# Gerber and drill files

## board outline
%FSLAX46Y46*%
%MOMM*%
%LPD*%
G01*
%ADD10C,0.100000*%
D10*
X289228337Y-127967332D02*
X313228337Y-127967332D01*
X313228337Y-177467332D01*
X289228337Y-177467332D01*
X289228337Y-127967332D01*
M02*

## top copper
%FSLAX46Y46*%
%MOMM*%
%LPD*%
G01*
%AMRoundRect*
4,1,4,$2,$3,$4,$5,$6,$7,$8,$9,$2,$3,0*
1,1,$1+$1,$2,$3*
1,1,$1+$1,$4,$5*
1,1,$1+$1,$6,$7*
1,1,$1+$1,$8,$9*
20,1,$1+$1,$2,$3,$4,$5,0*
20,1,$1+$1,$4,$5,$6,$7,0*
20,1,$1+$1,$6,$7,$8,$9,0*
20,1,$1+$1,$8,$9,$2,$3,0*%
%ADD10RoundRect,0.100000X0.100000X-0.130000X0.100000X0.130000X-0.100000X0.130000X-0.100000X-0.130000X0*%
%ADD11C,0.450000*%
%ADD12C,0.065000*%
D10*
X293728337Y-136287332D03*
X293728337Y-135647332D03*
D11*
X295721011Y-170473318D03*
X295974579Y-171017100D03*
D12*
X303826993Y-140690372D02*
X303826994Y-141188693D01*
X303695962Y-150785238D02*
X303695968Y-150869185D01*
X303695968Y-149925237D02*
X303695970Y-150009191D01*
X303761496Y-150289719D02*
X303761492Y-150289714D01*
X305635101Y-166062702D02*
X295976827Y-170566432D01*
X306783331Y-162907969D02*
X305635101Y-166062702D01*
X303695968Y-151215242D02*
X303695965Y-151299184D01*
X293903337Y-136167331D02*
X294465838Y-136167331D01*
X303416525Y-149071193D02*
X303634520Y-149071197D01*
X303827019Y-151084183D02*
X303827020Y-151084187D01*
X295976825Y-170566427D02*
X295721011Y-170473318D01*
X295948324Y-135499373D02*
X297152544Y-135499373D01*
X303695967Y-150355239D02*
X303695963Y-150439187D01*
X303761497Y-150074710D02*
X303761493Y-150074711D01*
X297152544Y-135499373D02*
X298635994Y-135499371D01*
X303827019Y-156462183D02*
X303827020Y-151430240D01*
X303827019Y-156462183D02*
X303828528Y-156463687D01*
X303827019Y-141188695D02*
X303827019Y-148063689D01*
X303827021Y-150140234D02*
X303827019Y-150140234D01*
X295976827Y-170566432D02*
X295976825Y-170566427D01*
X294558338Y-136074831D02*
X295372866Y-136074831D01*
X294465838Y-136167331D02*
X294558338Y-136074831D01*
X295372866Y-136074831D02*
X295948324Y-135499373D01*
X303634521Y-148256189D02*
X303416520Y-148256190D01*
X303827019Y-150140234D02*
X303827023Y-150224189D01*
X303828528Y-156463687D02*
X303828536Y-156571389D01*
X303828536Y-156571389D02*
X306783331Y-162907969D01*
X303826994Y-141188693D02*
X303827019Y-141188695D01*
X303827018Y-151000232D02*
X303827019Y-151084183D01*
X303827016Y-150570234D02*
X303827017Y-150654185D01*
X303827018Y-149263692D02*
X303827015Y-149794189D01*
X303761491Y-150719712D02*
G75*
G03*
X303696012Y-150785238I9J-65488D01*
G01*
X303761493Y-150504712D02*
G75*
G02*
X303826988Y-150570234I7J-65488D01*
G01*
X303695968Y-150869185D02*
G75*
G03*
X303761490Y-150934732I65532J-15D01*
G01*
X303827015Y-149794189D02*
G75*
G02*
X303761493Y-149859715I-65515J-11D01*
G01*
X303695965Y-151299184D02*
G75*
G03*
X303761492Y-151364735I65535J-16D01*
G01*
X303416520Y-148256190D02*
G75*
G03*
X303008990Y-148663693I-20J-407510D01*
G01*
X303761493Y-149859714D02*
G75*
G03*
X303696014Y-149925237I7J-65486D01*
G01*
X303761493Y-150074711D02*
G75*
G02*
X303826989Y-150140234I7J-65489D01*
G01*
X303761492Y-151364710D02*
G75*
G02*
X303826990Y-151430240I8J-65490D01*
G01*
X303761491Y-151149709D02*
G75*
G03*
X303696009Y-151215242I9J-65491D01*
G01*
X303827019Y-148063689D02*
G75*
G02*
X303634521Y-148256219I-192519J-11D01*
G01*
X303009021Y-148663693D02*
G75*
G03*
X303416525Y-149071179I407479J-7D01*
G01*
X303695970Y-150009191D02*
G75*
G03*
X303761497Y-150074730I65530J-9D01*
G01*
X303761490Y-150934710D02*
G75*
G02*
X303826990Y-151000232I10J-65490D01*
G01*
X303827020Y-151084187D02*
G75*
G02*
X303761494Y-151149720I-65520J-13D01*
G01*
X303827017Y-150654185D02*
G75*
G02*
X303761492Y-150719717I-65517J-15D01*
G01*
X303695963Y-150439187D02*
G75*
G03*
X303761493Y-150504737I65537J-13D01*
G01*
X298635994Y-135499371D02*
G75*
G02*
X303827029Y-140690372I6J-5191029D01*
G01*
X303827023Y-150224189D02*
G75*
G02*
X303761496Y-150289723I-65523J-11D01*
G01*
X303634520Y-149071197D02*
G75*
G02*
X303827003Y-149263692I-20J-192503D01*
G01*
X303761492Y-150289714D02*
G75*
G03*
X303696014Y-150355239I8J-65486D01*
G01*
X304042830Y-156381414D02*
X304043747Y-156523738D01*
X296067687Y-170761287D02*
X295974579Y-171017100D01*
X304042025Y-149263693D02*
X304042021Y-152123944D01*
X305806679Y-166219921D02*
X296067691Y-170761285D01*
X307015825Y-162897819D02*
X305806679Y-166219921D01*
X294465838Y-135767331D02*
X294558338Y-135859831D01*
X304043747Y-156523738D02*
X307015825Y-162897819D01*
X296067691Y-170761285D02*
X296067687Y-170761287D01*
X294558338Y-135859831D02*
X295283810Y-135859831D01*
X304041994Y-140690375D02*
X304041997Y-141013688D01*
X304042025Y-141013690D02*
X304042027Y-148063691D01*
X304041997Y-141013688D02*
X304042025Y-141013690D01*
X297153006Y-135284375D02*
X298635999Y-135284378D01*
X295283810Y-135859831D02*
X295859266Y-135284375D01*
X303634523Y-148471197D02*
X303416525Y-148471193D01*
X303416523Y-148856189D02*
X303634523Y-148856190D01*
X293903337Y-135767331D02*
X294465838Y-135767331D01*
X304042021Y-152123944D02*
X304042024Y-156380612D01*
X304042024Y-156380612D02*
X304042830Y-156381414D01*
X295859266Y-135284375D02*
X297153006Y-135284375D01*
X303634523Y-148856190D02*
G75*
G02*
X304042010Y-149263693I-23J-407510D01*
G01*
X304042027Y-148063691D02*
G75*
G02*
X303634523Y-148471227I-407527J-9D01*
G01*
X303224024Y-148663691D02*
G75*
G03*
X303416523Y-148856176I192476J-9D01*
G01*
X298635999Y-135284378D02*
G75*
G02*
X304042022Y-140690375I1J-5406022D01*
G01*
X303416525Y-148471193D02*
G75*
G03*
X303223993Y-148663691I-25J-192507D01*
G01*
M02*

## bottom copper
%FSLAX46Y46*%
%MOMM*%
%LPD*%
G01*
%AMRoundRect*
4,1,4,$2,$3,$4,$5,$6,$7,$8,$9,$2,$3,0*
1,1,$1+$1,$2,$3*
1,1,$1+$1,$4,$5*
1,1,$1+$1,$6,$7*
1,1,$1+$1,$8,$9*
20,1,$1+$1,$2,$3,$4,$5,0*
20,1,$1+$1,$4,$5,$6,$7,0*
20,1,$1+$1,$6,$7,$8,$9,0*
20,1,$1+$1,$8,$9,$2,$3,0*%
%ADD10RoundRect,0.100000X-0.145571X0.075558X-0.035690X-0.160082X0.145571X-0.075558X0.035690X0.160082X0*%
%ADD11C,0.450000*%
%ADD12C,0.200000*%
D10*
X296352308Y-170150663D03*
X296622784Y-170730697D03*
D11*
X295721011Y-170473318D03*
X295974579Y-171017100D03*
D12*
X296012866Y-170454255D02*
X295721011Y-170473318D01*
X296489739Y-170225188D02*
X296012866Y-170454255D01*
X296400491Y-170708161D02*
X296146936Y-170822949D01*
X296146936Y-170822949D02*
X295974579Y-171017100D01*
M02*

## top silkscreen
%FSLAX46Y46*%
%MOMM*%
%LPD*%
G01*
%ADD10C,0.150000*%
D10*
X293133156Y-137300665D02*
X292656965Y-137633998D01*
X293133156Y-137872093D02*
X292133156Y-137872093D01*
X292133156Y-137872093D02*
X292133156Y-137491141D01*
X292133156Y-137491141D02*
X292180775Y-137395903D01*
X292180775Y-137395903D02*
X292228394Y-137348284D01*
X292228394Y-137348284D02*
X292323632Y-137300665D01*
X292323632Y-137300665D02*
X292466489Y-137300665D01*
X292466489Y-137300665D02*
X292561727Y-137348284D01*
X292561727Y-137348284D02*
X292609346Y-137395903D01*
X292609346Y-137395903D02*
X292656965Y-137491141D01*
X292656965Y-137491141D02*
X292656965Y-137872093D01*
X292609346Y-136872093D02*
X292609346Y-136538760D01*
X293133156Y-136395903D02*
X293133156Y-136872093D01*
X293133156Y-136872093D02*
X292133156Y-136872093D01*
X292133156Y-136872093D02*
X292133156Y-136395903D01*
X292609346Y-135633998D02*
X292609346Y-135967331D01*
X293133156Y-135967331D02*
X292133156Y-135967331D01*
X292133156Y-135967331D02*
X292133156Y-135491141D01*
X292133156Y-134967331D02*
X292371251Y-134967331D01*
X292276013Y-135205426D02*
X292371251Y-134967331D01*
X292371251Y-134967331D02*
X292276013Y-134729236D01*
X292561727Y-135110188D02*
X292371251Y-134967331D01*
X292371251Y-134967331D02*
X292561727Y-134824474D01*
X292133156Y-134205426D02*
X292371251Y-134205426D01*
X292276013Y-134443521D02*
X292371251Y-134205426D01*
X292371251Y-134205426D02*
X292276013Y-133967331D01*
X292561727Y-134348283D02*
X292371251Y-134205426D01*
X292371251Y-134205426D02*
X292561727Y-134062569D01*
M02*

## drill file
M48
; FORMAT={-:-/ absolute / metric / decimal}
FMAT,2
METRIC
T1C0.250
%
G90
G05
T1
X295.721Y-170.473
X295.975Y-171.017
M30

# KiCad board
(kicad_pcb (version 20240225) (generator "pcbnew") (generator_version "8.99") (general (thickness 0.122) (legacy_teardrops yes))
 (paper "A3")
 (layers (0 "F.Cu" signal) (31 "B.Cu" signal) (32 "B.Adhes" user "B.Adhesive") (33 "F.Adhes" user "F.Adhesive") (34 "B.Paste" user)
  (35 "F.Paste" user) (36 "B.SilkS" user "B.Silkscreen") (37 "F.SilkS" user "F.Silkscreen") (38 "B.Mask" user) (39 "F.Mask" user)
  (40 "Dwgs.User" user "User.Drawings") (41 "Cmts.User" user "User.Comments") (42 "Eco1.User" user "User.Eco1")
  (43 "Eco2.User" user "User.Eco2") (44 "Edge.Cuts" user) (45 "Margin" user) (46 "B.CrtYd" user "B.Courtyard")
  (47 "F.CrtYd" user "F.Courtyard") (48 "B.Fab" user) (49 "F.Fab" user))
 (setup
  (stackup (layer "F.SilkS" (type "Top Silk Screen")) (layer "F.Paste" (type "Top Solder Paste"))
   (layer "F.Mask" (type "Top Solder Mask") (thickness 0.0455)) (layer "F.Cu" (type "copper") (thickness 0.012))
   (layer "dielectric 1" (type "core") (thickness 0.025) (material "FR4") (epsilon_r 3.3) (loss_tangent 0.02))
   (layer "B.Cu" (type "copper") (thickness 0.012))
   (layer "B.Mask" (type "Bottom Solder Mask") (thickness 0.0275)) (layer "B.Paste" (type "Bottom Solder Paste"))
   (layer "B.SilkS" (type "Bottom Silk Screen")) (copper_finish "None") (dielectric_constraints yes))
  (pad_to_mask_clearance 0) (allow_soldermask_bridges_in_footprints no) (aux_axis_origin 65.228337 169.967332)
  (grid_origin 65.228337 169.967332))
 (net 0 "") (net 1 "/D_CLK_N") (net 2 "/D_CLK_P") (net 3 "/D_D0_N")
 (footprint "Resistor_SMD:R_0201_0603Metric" (layer "F.Cu") (at 293.728337 135.967332 90)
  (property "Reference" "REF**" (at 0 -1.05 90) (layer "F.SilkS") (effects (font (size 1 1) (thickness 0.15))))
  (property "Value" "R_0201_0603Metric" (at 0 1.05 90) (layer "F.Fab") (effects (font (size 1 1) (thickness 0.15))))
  (pad "" smd roundrect (at -0.345 0 90) (size 0.318 0.36) (layers "F.Paste") (roundrect_rratio 0.25))
  (pad "" smd roundrect (at 0.345 0 90) (size 0.318 0.36) (layers "F.Paste") (roundrect_rratio 0.25))
  (pad "1" smd roundrect (at -0.32 0 90) (size 0.46 0.4) (layers "F.Cu" "F.Mask") (roundrect_rratio 0.25) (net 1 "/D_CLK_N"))
  (pad "2" smd roundrect (at 0.32 0 90) (size 0.46 0.4) (layers "F.Cu" "F.Mask") (roundrect_rratio 0.25) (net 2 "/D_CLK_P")))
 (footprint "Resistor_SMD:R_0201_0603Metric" (layer "B.Cu") (at 296.487546 170.44068 -65)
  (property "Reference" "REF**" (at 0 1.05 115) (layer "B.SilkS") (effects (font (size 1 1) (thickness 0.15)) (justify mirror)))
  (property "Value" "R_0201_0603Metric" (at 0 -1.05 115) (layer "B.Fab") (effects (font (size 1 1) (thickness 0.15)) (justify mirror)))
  (pad "" smd roundrect (at -0.345001 -0.000001 295) (size 0.318 0.36) (layers "B.Paste") (roundrect_rratio 0.25))
  (pad "" smd roundrect (at 0.345001 0.000001 295) (size 0.318 0.36) (layers "B.Paste") (roundrect_rratio 0.25))
  (pad "1" smd roundrect (at -0.319999 0.000001 295) (size 0.46 0.4) (layers "B.Cu" "B.Mask") (roundrect_rratio 0.25) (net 1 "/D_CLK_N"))
  (pad "2" smd roundrect (at 0.319999 -0.000001 295) (size 0.46 0.4) (layers "B.Cu" "B.Mask") (roundrect_rratio 0.25) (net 2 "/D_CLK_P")))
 (gr_rect (start 289.228337 127.967332) (end 313.228337 177.467332) (stroke (width 0.1) (type default)) (fill none) (layer "Edge.Cuts"))
 (segment (start 303.826993 140.690372) (end 303.826994 141.188693) (width 0.065) (layer "F.Cu") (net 1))
 (segment (start 303.695962 150.785238) (end 303.695968 150.869185) (width 0.065) (layer "F.Cu") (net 1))
 (segment (start 303.695968 149.925237) (end 303.69597 150.009191) (width 0.065) (layer "F.Cu") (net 1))
 (segment (start 303.761496 150.289719) (end 303.761492 150.289714) (width 0.065) (layer "F.Cu") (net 1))
 (segment (start 305.635101 166.062702) (end 295.976827 170.566432) (width 0.065) (layer "F.Cu") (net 1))
 (segment (start 306.783331 162.907969) (end 305.635101 166.062702) (width 0.065) (layer "F.Cu") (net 1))
 (segment (start 303.695968 151.215242) (end 303.695965 151.299184) (width 0.065) (layer "F.Cu") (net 1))
 (segment (start 293.903337 136.167331) (end 294.465838 136.167331) (width 0.065) (layer "F.Cu") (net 1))
 (segment (start 303.416525 149.071193) (end 303.63452 149.071197) (width 0.065) (layer "F.Cu") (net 1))
 (segment (start 303.827019 151.084183) (end 303.82702 151.084187) (width 0.065) (layer "F.Cu") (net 1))
 (segment (start 295.976825 170.566427) (end 295.721011 170.473318) (width 0.065) (layer "F.Cu") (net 1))
 (segment (start 295.948324 135.499373) (end 297.152544 135.499373) (width 0.065) (layer "F.Cu") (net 1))
 (segment (start 303.695967 150.355239) (end 303.695963 150.439187) (width 0.065) (layer "F.Cu") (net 1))
 (segment (start 303.761497 150.07471) (end 303.761493 150.074711) (width 0.065) (layer "F.Cu") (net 1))
 (segment (start 297.152544 135.499373) (end 298.635994 135.499371) (width 0.065) (layer "F.Cu") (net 1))
 (segment (start 303.827019 156.462183) (end 303.82702 151.43024) (width 0.065) (layer "F.Cu") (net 1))
 (segment (start 303.827019 156.462183) (end 303.828528 156.463687) (width 0.065) (layer "F.Cu") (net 1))
 (segment (start 303.827019 141.188695) (end 303.827019 148.063689) (width 0.065) (layer "F.Cu") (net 1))
 (segment (start 303.827021 150.140234) (end 303.827019 150.140234) (width 0.065) (layer "F.Cu") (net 1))
 (segment (start 295.976827 170.566432) (end 295.976825 170.566427) (width 0.065) (layer "F.Cu") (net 1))
 (segment (start 294.558338 136.074831) (end 295.372866 136.074831) (width 0.065) (layer "F.Cu") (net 1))
 (segment (start 294.465838 136.167331) (end 294.558338 136.074831) (width 0.065) (layer "F.Cu") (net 1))
 (segment (start 295.372866 136.074831) (end 295.948324 135.499373) (width 0.065) (layer "F.Cu") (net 1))
 (segment (start 303.634521 148.256189) (end 303.41652 148.25619) (width 0.065) (layer "F.Cu") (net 1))
 (segment (start 303.827019 150.140234) (end 303.827023 150.224189) (width 0.065) (layer "F.Cu") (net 1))
 (segment (start 303.828528 156.463687) (end 303.828536 156.571389) (width 0.065) (layer "F.Cu") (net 1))
 (segment (start 303.828536 156.571389) (end 306.783331 162.907969) (width 0.065) (layer "F.Cu") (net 1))
 (segment (start 303.826994 141.188693) (end 303.827019 141.188695) (width 0.065) (layer "F.Cu") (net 1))
 (segment (start 303.827018 151.000232) (end 303.827019 151.084183) (width 0.065) (layer "F.Cu") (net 1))
 (segment (start 303.827016 150.570234) (end 303.827017 150.654185) (width 0.065) (layer "F.Cu") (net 1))
 (segment (start 303.827018 149.263692) (end 303.827015 149.794189) (width 0.065) (layer "F.Cu") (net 1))
 (via (at 295.721011 170.473318) (size 0.45) (drill 0.25) (layers "F.Cu" "B.Cu") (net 1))
 (arc (start 303.761491 150.719712) (mid 303.715159 150.7389) (end 303.695962 150.785238) (width 0.065) (layer "F.Cu") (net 1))
 (arc (start 303.761493 150.504712) (mid 303.807829 150.523902) (end 303.827016 150.570234) (width 0.065) (layer "F.Cu") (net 1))
 (arc (start 303.695968 150.869185) (mid 303.715158 150.915521) (end 303.76149 150.93471) (width 0.065) (layer "F.Cu") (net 1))
 (arc (start 303.827015 149.794189) (mid 303.807827 149.840523) (end 303.761493 149.859714) (width 0.065) (layer "F.Cu") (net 1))
 (arc (start 303.695965 151.299184) (mid 303.715157 151.34552) (end 303.761492 151.36471) (width 0.065) (layer "F.Cu") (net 1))
 (arc (start 303.41652 148.25619) (mid 303.128372 148.375544) (end 303.009021 148.663693) (width 0.065) (layer "F.Cu") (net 1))
 (arc (start 303.761493 149.859714) (mid 303.715161 149.878904) (end 303.695968 149.925237) (width 0.065) (layer "F.Cu") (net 1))
 (arc (start 303.761493 150.074711) (mid 303.807826 150.093904) (end 303.827021 150.140234) (width 0.065) (layer "F.Cu") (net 1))
 (arc (start 303.761492 151.36471) (mid 303.807826 151.383901) (end 303.82702 151.43024) (width 0.065) (layer "F.Cu") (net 1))
 (arc (start 303.761491 151.149709) (mid 303.715157 151.168904) (end 303.695968 151.215242) (width 0.065) (layer "F.Cu") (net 1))
 (arc (start 303.827019 148.063689) (mid 303.770636 148.199803) (end 303.634521 148.256189) (width 0.065) (layer "F.Cu") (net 1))
 (arc (start 303.009021 148.663693) (mid 303.128374 148.951835) (end 303.416525 149.071193) (width 0.065) (layer "F.Cu") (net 1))
 (arc (start 303.69597 150.009191) (mid 303.715165 150.055521) (end 303.761497 150.07471) (width 0.065) (layer "F.Cu") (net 1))
 (arc (start 303.76149 150.93471) (mid 303.807827 150.953903) (end 303.827018 151.000232) (width 0.065) (layer "F.Cu") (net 1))
 (arc (start 303.82702 151.084187) (mid 303.807825 151.130523) (end 303.761494 151.149711) (width 0.065) (layer "F.Cu") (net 1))
 (arc (start 303.827017 150.654185) (mid 303.807827 150.700522) (end 303.761492 150.719716) (width 0.065) (layer "F.Cu") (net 1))
 (arc (start 303.695963 150.439187) (mid 303.715156 150.485523) (end 303.761493 150.504712) (width 0.065) (layer "F.Cu") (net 1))
 (arc (start 298.635994 135.499371) (mid 302.306582 137.019788) (end 303.826993 140.690372) (width 0.065) (layer "F.Cu") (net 1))
 (arc (start 303.827023 150.224189) (mid 303.80783 150.270521) (end 303.761496 150.289719) (width 0.065) (layer "F.Cu") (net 1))
 (arc (start 303.63452 149.071197) (mid 303.770637 149.127573) (end 303.827018 149.263692) (width 0.065) (layer "F.Cu") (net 1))
 (arc (start 303.761492 150.289714) (mid 303.715158 150.308906) (end 303.695967 150.355239) (width 0.065) (layer "F.Cu") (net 1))
 (segment (start 296.012866 170.454255) (end 295.721011 170.473318) (width 0.2) (layer "B.Cu") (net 1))
 (segment (start 296.489739 170.225188) (end 296.012866 170.454255) (width 0.2) (layer "B.Cu") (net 1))
 (segment (start 304.04283 156.381414) (end 304.043747 156.523738) (width 0.065) (layer "F.Cu") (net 2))
 (segment (start 296.067687 170.761287) (end 295.974579 171.0171) (width 0.065) (layer "F.Cu") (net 2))
 (segment (start 304.042025 149.263693) (end 304.042021 152.123944) (width 0.065) (layer "F.Cu") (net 2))
 (segment (start 305.806679 166.219921) (end 296.067691 170.761285) (width 0.065) (layer "F.Cu") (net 2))
 (segment (start 307.015825 162.897819) (end 305.806679 166.219921) (width 0.065) (layer "F.Cu") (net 2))
 (segment (start 294.465838 135.767331) (end 294.558338 135.859831) (width 0.065) (layer "F.Cu") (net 2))
 (segment (start 304.043747 156.523738) (end 307.015825 162.897819) (width 0.065) (layer "F.Cu") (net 2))
 (segment (start 296.067691 170.761285) (end 296.067687 170.761287) (width 0.065) (layer "F.Cu") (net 2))
 (segment (start 294.558338 135.859831) (end 295.28381 135.859831) (width 0.065) (layer "F.Cu") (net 2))
 (segment (start 304.041994 140.690375) (end 304.041997 141.013688) (width 0.065) (layer "F.Cu") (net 2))
 (segment (start 304.042025 141.01369) (end 304.042027 148.063691) (width 0.065) (layer "F.Cu") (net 2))
 (segment (start 304.041997 141.013688) (end 304.042025 141.01369) (width 0.065) (layer "F.Cu") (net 2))
 (segment (start 297.153006 135.284375) (end 298.635999 135.284378) (width 0.065) (layer "F.Cu") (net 2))
 (segment (start 295.28381 135.859831) (end 295.859266 135.284375) (width 0.065) (layer "F.Cu") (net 2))
 (segment (start 303.634523 148.471197) (end 303.416525 148.471193) (width 0.065) (layer "F.Cu") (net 2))
 (segment (start 303.416523 148.856189) (end 303.634523 148.85619) (width 0.065) (layer "F.Cu") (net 2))
 (segment (start 293.903337 135.767331) (end 294.465838 135.767331) (width 0.065) (layer "F.Cu") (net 2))
 (segment (start 304.042021 152.123944) (end 304.042024 156.380612) (width 0.065) (layer "F.Cu") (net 2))
 (segment (start 304.042024 156.380612) (end 304.04283 156.381414) (width 0.065) (layer "F.Cu") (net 2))
 (segment (start 295.859266 135.284375) (end 297.153006 135.284375) (width 0.065) (layer "F.Cu") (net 2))
 (via (at 295.974579 171.0171) (size 0.45) (drill 0.25) (layers "F.Cu" "B.Cu") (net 2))
 (arc (start 303.634523 148.85619) (mid 303.922673 148.975543) (end 304.042025 149.263693) (width 0.065) (layer "F.Cu") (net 2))
 (arc (start 304.042027 148.063691) (mid 303.922669 148.351835) (end 303.634523 148.471197) (width 0.065) (layer "F.Cu") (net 2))
 (arc (start 303.224024 148.663691) (mid 303.280406 148.799808) (end 303.416523 148.856189) (width 0.065) (layer "F.Cu") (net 2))
 (arc (start 298.635999 135.284378) (mid 302.458614 136.867756) (end 304.041994 140.690375) (width 0.065) (layer "F.Cu") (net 2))
 (arc (start 303.416525 148.471193) (mid 303.280408 148.527574) (end 303.224024 148.663691) (width 0.065) (layer "F.Cu") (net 2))
 (segment (start 296.400491 170.708161) (end 296.146936 170.822949) (width 0.2) (layer "B.Cu") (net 2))
 (segment (start 296.146936 170.822949) (end 295.974579 171.0171) (width 0.2) (layer "B.Cu") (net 2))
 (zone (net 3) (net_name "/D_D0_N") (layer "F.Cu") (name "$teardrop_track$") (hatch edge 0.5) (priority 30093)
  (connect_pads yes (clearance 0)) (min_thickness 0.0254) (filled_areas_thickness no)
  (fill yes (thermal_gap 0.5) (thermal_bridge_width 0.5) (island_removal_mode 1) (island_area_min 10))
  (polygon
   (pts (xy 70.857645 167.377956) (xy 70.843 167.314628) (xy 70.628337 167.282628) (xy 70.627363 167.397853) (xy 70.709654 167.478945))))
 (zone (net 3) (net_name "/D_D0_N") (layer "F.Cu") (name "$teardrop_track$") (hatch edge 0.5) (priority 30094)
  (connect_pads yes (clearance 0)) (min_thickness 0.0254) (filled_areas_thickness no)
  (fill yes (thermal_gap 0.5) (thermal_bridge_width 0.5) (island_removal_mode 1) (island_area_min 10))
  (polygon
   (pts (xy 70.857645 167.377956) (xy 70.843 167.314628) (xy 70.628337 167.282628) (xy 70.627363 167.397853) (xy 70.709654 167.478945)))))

